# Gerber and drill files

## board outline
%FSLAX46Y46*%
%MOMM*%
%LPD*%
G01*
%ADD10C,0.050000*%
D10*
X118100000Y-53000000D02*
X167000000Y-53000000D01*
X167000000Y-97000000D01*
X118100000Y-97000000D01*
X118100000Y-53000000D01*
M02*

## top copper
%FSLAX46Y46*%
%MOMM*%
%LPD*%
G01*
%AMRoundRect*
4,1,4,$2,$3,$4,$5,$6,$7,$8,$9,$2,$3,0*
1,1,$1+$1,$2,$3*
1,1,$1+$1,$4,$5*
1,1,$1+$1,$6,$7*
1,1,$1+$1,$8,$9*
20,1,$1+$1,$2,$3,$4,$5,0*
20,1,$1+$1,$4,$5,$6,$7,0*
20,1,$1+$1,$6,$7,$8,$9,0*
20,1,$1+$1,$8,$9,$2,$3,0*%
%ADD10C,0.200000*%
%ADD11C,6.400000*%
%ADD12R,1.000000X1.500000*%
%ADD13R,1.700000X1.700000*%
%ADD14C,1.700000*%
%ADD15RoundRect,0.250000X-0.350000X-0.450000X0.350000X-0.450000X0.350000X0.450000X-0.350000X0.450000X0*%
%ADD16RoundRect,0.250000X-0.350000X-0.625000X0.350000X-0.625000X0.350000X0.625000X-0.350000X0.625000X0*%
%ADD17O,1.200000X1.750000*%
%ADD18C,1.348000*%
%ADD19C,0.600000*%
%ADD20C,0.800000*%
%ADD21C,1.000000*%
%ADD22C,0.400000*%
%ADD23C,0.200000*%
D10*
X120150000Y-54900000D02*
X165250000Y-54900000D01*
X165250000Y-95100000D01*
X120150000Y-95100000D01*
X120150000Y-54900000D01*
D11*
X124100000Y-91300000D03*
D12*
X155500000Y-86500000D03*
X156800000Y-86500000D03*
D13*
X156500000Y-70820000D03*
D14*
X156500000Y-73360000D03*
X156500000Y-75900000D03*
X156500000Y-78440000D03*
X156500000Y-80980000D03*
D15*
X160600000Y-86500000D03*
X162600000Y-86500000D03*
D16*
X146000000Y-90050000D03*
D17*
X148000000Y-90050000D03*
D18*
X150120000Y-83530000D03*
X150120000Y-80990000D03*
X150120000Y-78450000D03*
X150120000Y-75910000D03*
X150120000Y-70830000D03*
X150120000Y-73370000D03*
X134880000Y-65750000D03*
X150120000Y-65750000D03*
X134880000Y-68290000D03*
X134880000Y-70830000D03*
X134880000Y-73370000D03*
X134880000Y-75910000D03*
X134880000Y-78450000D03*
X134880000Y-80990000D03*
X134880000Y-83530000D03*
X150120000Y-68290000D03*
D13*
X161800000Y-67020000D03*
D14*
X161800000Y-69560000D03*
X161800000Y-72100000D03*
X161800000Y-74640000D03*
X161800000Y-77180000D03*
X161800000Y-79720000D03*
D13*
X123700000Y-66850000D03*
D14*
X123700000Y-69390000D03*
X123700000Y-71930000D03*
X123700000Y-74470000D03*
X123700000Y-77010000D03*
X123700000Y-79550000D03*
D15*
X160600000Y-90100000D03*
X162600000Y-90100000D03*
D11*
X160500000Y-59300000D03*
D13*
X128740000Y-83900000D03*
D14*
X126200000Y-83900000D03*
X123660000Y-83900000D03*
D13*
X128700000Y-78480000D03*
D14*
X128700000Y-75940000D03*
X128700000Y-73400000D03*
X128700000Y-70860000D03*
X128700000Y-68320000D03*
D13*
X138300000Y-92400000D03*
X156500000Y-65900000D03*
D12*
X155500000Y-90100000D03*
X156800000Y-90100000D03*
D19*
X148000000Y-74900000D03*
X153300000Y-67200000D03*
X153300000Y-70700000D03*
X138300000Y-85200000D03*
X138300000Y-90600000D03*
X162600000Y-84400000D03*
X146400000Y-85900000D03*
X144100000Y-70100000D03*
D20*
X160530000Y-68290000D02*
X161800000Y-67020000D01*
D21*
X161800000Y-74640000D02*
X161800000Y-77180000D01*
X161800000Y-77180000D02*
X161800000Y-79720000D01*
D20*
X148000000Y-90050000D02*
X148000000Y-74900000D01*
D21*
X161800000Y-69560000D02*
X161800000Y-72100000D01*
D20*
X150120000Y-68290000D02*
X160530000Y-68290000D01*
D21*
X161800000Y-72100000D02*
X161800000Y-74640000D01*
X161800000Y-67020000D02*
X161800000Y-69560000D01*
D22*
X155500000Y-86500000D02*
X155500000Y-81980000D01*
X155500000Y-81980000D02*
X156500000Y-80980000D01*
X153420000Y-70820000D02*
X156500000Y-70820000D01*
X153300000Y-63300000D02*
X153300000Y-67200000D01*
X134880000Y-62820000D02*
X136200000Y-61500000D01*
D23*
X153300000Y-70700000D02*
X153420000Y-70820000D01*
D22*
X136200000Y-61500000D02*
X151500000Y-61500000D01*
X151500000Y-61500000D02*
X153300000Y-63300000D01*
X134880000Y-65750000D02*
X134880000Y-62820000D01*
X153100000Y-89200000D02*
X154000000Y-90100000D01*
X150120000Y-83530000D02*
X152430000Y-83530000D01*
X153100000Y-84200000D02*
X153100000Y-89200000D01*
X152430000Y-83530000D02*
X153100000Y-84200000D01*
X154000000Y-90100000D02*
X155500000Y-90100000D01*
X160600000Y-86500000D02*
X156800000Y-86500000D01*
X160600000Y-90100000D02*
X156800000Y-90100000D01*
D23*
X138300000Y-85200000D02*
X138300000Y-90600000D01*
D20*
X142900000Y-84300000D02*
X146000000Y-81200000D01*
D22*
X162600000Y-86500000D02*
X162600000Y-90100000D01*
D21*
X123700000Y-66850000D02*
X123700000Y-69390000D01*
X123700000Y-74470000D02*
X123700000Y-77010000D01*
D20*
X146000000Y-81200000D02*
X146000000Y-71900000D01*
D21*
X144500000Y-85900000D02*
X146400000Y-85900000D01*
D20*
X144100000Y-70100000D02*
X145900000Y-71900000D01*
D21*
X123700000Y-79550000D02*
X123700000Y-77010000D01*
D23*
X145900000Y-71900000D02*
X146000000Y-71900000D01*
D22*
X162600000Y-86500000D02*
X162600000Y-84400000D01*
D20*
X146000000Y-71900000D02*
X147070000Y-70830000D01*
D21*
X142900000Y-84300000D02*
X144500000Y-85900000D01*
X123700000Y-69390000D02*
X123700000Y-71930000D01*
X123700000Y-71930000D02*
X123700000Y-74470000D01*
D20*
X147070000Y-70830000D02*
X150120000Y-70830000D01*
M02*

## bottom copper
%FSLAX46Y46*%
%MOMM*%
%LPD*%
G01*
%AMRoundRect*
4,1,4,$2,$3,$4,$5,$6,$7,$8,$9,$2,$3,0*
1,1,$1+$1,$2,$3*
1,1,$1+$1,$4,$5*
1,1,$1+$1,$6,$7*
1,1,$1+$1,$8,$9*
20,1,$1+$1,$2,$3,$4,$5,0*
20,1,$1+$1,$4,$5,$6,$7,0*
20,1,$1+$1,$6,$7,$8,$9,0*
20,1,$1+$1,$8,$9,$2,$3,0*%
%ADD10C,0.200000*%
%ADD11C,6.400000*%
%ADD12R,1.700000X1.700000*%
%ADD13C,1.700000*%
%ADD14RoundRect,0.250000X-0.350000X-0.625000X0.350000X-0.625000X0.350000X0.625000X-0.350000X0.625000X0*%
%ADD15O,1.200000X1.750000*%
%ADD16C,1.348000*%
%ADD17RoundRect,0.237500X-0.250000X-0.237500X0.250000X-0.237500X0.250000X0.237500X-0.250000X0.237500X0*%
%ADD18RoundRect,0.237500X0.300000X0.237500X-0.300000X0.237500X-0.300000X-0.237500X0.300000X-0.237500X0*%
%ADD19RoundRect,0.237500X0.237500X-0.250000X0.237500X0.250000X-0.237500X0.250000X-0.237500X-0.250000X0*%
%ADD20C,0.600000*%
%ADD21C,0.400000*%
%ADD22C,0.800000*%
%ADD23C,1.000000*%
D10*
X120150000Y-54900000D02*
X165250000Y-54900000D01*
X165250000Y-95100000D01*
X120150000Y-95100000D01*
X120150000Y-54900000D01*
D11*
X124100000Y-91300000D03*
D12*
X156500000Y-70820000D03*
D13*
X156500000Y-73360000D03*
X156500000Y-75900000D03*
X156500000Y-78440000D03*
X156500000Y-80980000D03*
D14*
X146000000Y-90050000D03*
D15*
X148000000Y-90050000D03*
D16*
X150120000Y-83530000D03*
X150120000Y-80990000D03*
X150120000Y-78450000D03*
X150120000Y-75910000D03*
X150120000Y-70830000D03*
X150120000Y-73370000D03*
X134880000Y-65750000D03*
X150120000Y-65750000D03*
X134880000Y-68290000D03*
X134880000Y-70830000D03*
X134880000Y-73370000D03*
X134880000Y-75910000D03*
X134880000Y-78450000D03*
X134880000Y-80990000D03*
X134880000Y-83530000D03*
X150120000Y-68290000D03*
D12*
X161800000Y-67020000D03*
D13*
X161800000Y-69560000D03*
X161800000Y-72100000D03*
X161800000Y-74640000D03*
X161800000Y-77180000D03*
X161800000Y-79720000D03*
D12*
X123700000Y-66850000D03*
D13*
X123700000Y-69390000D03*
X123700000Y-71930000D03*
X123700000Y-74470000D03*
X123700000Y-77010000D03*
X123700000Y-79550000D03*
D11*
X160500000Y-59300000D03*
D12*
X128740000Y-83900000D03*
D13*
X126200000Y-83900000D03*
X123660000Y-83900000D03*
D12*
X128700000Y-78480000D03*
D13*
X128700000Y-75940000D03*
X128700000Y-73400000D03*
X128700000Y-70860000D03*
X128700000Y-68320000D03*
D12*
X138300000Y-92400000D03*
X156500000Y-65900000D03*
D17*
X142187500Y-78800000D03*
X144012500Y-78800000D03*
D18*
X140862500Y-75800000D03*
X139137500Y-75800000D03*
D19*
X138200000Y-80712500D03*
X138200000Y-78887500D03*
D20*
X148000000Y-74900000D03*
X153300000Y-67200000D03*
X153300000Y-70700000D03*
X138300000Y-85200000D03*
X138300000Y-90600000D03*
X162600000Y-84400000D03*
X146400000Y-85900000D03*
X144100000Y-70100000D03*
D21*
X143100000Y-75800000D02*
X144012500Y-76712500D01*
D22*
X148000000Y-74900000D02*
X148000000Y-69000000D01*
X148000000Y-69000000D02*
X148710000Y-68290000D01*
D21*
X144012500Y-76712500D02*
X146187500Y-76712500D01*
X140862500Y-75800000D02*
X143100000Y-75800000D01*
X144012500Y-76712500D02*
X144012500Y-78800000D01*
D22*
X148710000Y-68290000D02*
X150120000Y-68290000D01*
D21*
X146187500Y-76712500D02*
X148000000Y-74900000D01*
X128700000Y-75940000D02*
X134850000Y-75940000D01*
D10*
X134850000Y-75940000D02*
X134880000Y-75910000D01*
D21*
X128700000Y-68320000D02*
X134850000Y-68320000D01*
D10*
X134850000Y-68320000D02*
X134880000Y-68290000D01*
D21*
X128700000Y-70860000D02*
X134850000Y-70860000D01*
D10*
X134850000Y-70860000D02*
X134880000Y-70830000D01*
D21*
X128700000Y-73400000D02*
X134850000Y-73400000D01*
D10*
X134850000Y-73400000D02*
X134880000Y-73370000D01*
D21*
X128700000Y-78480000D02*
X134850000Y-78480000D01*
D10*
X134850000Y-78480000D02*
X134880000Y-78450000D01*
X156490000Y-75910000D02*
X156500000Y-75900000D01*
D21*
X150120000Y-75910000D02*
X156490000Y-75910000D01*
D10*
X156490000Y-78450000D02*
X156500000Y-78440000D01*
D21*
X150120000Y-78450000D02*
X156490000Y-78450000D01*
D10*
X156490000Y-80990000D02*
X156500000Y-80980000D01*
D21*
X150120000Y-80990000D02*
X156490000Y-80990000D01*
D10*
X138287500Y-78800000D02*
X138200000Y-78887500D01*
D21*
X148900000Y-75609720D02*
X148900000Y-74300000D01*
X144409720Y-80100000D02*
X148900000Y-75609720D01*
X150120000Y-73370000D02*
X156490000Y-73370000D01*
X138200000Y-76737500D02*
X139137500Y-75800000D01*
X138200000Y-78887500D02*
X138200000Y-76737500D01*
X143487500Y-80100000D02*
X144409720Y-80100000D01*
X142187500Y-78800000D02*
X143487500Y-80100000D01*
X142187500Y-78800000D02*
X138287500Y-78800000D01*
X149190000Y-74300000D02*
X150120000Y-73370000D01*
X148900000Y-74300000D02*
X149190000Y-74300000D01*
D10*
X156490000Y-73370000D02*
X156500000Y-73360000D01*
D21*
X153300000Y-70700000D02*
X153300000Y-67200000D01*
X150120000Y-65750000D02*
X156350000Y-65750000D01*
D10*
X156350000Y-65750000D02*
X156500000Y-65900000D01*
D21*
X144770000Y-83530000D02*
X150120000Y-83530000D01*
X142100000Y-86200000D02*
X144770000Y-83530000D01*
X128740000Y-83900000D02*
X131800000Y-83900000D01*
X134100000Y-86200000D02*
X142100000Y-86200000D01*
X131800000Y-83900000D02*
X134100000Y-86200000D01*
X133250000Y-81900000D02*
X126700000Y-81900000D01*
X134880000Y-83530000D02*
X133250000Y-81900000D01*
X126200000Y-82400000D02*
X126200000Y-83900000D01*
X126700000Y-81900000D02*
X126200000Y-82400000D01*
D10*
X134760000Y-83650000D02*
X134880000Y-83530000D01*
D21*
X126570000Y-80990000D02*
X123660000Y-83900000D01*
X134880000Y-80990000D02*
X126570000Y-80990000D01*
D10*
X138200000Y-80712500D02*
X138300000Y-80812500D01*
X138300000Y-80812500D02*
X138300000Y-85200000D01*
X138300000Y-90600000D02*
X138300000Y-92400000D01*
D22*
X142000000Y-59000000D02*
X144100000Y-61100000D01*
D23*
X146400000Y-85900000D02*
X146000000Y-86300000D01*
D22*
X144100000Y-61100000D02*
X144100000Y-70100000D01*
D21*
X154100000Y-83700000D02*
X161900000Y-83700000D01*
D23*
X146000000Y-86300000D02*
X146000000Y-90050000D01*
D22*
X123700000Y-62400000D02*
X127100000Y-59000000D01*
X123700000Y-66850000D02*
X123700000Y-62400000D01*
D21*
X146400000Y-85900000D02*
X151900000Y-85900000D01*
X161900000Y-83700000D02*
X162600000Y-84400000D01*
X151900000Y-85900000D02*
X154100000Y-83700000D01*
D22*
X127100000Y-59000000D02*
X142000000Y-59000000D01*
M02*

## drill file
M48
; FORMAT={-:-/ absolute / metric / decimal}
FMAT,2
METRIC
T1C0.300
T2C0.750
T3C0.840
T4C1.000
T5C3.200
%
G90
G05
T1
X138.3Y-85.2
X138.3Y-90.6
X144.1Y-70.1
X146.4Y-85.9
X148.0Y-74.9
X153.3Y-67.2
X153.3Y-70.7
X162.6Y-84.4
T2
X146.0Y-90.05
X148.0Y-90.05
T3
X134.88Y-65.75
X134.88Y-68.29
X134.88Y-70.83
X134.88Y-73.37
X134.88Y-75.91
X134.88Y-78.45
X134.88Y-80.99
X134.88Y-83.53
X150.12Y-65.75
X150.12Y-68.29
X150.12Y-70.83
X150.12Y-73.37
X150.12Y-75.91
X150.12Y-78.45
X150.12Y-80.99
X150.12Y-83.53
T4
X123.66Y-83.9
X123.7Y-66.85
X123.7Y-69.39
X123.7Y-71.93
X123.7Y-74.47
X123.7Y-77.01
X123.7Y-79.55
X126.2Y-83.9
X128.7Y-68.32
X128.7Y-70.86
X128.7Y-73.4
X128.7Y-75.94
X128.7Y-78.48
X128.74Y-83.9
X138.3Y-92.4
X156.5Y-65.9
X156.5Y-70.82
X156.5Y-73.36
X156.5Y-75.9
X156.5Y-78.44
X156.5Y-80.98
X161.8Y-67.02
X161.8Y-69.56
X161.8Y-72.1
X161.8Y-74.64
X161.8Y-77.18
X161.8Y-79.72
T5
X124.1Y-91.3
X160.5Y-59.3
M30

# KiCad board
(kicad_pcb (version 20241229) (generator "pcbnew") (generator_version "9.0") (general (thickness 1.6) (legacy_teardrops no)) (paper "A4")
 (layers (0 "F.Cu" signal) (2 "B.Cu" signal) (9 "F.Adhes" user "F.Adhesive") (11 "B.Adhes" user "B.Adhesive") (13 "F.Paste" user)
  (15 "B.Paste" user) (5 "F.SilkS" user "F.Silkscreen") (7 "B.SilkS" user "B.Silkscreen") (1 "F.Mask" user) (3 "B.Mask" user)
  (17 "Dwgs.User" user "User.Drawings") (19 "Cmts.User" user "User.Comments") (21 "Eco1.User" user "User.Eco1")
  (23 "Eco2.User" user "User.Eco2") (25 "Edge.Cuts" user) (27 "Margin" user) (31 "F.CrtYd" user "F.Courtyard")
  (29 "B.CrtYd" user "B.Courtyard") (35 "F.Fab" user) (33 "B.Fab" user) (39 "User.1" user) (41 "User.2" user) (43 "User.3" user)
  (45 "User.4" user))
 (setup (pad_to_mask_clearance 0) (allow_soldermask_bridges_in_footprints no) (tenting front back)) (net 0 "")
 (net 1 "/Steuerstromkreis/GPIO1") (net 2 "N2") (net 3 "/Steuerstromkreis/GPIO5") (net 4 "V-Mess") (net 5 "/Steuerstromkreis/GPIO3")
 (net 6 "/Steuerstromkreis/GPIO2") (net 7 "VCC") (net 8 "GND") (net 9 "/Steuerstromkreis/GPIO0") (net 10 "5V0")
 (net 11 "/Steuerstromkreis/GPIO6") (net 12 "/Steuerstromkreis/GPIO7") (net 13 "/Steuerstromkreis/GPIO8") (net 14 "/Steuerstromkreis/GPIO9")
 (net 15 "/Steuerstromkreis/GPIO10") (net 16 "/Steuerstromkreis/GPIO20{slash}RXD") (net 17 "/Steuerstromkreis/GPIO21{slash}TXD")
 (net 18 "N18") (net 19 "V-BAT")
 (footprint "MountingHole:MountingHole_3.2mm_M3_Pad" (layer "F.Cu") (at 124.1 91.3)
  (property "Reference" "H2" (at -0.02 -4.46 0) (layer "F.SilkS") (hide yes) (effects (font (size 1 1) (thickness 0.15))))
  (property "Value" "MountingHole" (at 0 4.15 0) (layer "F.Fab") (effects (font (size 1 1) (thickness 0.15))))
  (pad "1" thru_hole circle (at 0 0) (size 6.4 6.4) (drill 3.2) (layers "*.Cu" "*.Mask") (remove_unused_layers no) (zone_connect 2)))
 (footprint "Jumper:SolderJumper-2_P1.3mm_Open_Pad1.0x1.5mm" (layer "F.Cu") (at 156.15 86.5)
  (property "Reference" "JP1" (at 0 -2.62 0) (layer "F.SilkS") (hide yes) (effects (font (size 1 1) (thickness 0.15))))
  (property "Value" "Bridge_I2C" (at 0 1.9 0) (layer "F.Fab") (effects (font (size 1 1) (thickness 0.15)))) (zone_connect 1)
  (pad "1" smd rect (at -0.65 0) (size 1 1.5) (layers "F.Cu" "F.Mask") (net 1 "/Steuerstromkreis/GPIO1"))
  (pad "2" smd rect (at 0.65 0) (size 1 1.5) (layers "F.Cu" "F.Mask") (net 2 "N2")))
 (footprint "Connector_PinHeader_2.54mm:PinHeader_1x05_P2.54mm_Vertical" (layer "F.Cu") (at 156.5 70.82)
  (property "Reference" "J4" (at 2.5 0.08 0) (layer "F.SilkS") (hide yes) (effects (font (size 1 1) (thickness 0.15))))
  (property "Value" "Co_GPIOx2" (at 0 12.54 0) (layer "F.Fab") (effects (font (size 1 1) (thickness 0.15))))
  (pad "1" thru_hole rect (at 0 0) (size 1.7 1.7) (drill 1) (layers "*.Cu" "*.Mask") (remove_unused_layers no)
   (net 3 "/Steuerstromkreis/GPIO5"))
  (pad "2" thru_hole circle (at 0 2.54) (size 1.7 1.7) (drill 1) (layers "*.Cu" "*.Mask") (remove_unused_layers no) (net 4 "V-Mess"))
  (pad "3" thru_hole circle (at 0 5.08) (size 1.7 1.7) (drill 1) (layers "*.Cu" "*.Mask") (remove_unused_layers no)
   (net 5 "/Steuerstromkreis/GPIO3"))
  (pad "4" thru_hole circle (at 0 7.62) (size 1.7 1.7) (drill 1) (layers "*.Cu" "*.Mask") (remove_unused_layers no)
   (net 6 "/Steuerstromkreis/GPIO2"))
  (pad "5" thru_hole circle (at 0 10.16) (size 1.7 1.7) (drill 1) (layers "*.Cu" "*.Mask") (remove_unused_layers no)
   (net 1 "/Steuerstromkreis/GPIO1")))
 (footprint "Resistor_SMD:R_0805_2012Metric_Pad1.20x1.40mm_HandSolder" (layer "F.Cu") (at 161.6 86.5)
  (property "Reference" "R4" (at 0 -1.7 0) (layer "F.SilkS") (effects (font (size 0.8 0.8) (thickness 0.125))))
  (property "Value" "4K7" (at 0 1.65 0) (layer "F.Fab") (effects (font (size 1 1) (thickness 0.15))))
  (pad "1" smd roundrect (at -1 0) (size 1.2 1.4) (layers "F.Cu" "F.Mask" "F.Paste") (roundrect_rratio 0.208333) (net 2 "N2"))
  (pad "2" smd roundrect (at 1 0) (size 1.2 1.4) (layers "F.Cu" "F.Mask" "F.Paste") (roundrect_rratio 0.208333) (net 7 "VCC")))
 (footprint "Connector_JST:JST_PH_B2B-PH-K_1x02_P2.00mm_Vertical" (layer "F.Cu") (at 146 90.05)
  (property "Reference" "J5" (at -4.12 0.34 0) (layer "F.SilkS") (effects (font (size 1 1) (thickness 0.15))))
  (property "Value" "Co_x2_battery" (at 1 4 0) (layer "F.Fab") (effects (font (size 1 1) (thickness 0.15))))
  (pad "1" thru_hole roundrect (at 0 0) (size 1.2 1.75) (drill 0.75) (layers "*.Cu" "*.Mask") (remove_unused_layers no)
   (roundrect_rratio 0.208333) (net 7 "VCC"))
  (pad "2" thru_hole oval (at 2 0) (size 1.2 1.75) (drill 0.75) (layers "*.Cu" "*.Mask") (remove_unused_layers no) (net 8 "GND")))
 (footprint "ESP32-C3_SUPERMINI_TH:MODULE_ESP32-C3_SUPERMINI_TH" (layer "F.Cu") (at 142.5 75.65)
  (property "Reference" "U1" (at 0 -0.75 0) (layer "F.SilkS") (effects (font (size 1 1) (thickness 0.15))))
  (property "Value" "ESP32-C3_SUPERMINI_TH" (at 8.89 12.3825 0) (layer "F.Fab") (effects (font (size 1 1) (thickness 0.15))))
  (pad "0" thru_hole circle (at 7.62 7.88) (size 1.348 1.348) (drill 0.84) (layers "*.Cu" "*.Mask") (remove_unused_layers no)
   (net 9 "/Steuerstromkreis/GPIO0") (solder_mask_margin 0.102))
  (pad "1" thru_hole circle (at 7.62 5.34) (size 1.348 1.348) (drill 0.84) (layers "*.Cu" "*.Mask") (remove_unused_layers no)
   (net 1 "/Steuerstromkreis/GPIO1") (solder_mask_margin 0.102))
  (pad "2" thru_hole circle (at 7.62 2.8) (size 1.348 1.348) (drill 0.84) (layers "*.Cu" "*.Mask") (remove_unused_layers no)
   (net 6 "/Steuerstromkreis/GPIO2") (solder_mask_margin 0.102))
  (pad "3" thru_hole circle (at 7.62 0.26) (size 1.348 1.348) (drill 0.84) (layers "*.Cu" "*.Mask") (remove_unused_layers no)
   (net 5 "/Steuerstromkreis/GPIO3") (solder_mask_margin 0.102))
  (pad "3.3" thru_hole circle (at 7.62 -4.82) (size 1.348 1.348) (drill 0.84) (layers "*.Cu" "*.Mask") (remove_unused_layers no)
   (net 7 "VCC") (solder_mask_margin 0.102))
  (pad "4" thru_hole circle (at 7.62 -2.28) (size 1.348 1.348) (drill 0.84) (layers "*.Cu" "*.Mask") (remove_unused_layers no)
   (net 4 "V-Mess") (solder_mask_margin 0.102))
  (pad "5" thru_hole circle (at -7.62 -9.9) (size 1.348 1.348) (drill 0.84) (layers "*.Cu" "*.Mask") (remove_unused_layers no)
   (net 3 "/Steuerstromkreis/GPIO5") (solder_mask_margin 0.102))
  (pad "5V" thru_hole circle (at 7.62 -9.9) (size 1.348 1.348) (drill 0.84) (layers "*.Cu" "*.Mask") (remove_unused_layers no)
   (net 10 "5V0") (solder_mask_margin 0.102))
  (pad "6" thru_hole circle (at -7.62 -7.36) (size 1.348 1.348) (drill 0.84) (layers "*.Cu" "*.Mask") (remove_unused_layers no)
   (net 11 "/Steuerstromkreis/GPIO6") (solder_mask_margin 0.102))
  (pad "7" thru_hole circle (at -7.62 -4.82) (size 1.348 1.348) (drill 0.84) (layers "*.Cu" "*.Mask") (remove_unused_layers no)
   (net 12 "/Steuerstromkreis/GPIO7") (solder_mask_margin 0.102))
  (pad "8" thru_hole circle (at -7.62 -2.28) (size 1.348 1.348) (drill 0.84) (layers "*.Cu" "*.Mask") (remove_unused_layers no)
   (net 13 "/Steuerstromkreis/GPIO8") (solder_mask_margin 0.102))
  (pad "9" thru_hole circle (at -7.62 0.26) (size 1.348 1.348) (drill 0.84) (layers "*.Cu" "*.Mask") (remove_unused_layers no)
   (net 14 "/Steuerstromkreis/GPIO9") (solder_mask_margin 0.102))
  (pad "10" thru_hole circle (at -7.62 2.8) (size 1.348 1.348) (drill 0.84) (layers "*.Cu" "*.Mask") (remove_unused_layers no)
   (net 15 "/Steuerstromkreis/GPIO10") (solder_mask_margin 0.102))
  (pad "20" thru_hole circle (at -7.62 5.34) (size 1.348 1.348) (drill 0.84) (layers "*.Cu" "*.Mask") (remove_unused_layers no)
   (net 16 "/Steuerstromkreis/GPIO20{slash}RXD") (solder_mask_margin 0.102))
  (pad "21" thru_hole circle (at -7.62 7.88) (size 1.348 1.348) (drill 0.84) (layers "*.Cu" "*.Mask") (remove_unused_layers no)
   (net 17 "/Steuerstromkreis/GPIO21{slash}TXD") (solder_mask_margin 0.102))
  (pad "G" thru_hole circle (at 7.62 -7.36) (size 1.348 1.348) (drill 0.84) (layers "*.Cu" "*.Mask") (remove_unused_layers no) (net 8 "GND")
   (solder_mask_margin 0.102)))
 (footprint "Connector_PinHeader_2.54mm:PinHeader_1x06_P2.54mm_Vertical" (layer "F.Cu") (at 161.8 67.02)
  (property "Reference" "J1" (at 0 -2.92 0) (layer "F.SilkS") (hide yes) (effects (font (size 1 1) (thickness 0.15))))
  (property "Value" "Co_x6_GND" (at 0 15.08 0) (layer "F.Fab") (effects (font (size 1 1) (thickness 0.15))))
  (pad "1" thru_hole rect (at 0 0) (size 1.7 1.7) (drill 1) (layers "*.Cu" "*.Mask") (remove_unused_layers no) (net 8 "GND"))
  (pad "2" thru_hole circle (at 0 2.54) (size 1.7 1.7) (drill 1) (layers "*.Cu" "*.Mask") (remove_unused_layers no) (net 8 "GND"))
  (pad "3" thru_hole circle (at 0 5.08) (size 1.7 1.7) (drill 1) (layers "*.Cu" "*.Mask") (remove_unused_layers no) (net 8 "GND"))
  (pad "4" thru_hole circle (at 0 7.62) (size 1.7 1.7) (drill 1) (layers "*.Cu" "*.Mask") (remove_unused_layers no) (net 8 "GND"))
  (pad "5" thru_hole circle (at 0 10.16) (size 1.7 1.7) (drill 1) (layers "*.Cu" "*.Mask") (remove_unused_layers no) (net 8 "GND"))
  (pad "6" thru_hole circle (at 0 12.7) (size 1.7 1.7) (drill 1) (layers "*.Cu" "*.Mask") (remove_unused_layers no) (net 8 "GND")))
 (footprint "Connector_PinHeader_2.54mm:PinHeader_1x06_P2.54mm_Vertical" (layer "F.Cu") (at 123.7 66.85)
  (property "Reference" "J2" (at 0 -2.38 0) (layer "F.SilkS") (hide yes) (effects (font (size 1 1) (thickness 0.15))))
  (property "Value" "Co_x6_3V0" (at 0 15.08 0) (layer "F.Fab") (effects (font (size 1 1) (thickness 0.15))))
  (pad "1" thru_hole rect (at 0 0) (size 1.7 1.7) (drill 1) (layers "*.Cu" "*.Mask") (remove_unused_layers no) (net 7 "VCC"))
  (pad "2" thru_hole circle (at 0 2.54) (size 1.7 1.7) (drill 1) (layers "*.Cu" "*.Mask") (remove_unused_layers no) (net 7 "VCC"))
  (pad "3" thru_hole circle (at 0 5.08) (size 1.7 1.7) (drill 1) (layers "*.Cu" "*.Mask") (remove_unused_layers no) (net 7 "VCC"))
  (pad "4" thru_hole circle (at 0 7.62) (size 1.7 1.7) (drill 1) (layers "*.Cu" "*.Mask") (remove_unused_layers no) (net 7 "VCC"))
  (pad "5" thru_hole circle (at 0 10.16) (size 1.7 1.7) (drill 1) (layers "*.Cu" "*.Mask") (remove_unused_layers no) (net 7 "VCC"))
  (pad "6" thru_hole circle (at 0 12.7) (size 1.7 1.7) (drill 1) (layers "*.Cu" "*.Mask") (remove_unused_layers no) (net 7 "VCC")))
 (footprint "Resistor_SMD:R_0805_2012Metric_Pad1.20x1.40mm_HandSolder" (layer "F.Cu") (at 161.6 90.1)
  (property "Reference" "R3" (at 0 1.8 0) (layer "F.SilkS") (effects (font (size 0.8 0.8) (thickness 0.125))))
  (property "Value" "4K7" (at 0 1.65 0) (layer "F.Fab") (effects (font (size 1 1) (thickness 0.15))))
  (pad "1" smd roundrect (at -1 0) (size 1.2 1.4) (layers "F.Cu" "F.Mask" "F.Paste") (roundrect_rratio 0.208333) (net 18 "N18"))
  (pad "2" smd roundrect (at 1 0) (size 1.2 1.4) (layers "F.Cu" "F.Mask" "F.Paste") (roundrect_rratio 0.208333) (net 7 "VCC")))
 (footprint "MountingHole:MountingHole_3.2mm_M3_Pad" (layer "F.Cu") (at 160.5 59.3)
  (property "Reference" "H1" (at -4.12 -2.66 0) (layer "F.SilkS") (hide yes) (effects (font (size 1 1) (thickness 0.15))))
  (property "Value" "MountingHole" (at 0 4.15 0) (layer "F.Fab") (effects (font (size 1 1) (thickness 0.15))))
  (pad "1" thru_hole circle (at 0 0) (size 6.4 6.4) (drill 3.2) (layers "*.Cu" "*.Mask") (remove_unused_layers no) (zone_connect 2)))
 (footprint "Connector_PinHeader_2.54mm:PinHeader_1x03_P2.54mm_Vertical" (layer "F.Cu") (at 128.74 83.9 -90)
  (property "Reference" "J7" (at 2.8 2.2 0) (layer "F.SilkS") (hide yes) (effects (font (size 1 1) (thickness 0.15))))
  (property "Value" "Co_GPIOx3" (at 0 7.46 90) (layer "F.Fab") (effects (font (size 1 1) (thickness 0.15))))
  (pad "1" thru_hole rect (at 0 0 270) (size 1.7 1.7) (drill 1) (layers "*.Cu" "*.Mask") (remove_unused_layers no)
   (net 9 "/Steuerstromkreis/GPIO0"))
  (pad "2" thru_hole circle (at 0 2.54 270) (size 1.7 1.7) (drill 1) (layers "*.Cu" "*.Mask") (remove_unused_layers no)
   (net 17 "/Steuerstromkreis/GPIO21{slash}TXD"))
  (pad "3" thru_hole circle (at 0 5.08 270) (size 1.7 1.7) (drill 1) (layers "*.Cu" "*.Mask") (remove_unused_layers no)
   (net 16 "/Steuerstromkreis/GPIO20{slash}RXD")))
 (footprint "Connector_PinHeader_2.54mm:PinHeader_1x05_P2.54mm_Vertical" (layer "F.Cu") (at 128.7 78.48 180)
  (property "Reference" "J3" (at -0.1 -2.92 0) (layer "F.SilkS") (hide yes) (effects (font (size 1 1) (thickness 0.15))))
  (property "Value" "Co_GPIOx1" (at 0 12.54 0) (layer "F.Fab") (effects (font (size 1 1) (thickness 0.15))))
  (pad "1" thru_hole rect (at 0 0 180) (size 1.7 1.7) (drill 1) (layers "*.Cu" "*.Mask") (remove_unused_layers no)
   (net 15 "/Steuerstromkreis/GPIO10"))
  (pad "2" thru_hole circle (at 0 2.54 180) (size 1.7 1.7) (drill 1) (layers "*.Cu" "*.Mask") (remove_unused_layers no)
   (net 14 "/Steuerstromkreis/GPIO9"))
  (pad "3" thru_hole circle (at 0 5.08 180) (size 1.7 1.7) (drill 1) (layers "*.Cu" "*.Mask") (remove_unused_layers no)
   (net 13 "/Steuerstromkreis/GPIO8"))
  (pad "4" thru_hole circle (at 0 7.62 180) (size 1.7 1.7) (drill 1) (layers "*.Cu" "*.Mask") (remove_unused_layers no)
   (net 12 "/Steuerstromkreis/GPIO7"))
  (pad "5" thru_hole circle (at 0 10.16 180) (size 1.7 1.7) (drill 1) (layers "*.Cu" "*.Mask") (remove_unused_layers no)
   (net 11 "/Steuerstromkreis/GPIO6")))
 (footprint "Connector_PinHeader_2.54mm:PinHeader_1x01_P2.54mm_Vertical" (layer "F.Cu") (at 138.3 92.4)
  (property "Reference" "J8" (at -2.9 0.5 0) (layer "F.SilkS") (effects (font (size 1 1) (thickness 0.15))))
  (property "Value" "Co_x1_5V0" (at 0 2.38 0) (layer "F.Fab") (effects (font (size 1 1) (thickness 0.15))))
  (pad "1" thru_hole rect (at 0 0) (size 1.7 1.7) (drill 1) (layers "*.Cu" "*.Mask") (remove_unused_layers no) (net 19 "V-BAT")))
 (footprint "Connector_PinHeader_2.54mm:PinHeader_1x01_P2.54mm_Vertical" (layer "F.Cu") (at 156.5 65.9)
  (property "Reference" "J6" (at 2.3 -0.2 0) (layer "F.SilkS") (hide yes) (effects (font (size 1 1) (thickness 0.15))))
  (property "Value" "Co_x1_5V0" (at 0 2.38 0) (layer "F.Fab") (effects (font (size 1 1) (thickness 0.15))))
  (pad "1" thru_hole rect (at 0 0) (size 1.7 1.7) (drill 1) (layers "*.Cu" "*.Mask") (remove_unused_layers no) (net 10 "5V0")))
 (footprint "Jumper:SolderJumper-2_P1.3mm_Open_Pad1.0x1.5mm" (layer "F.Cu") (at 156.15 90.1)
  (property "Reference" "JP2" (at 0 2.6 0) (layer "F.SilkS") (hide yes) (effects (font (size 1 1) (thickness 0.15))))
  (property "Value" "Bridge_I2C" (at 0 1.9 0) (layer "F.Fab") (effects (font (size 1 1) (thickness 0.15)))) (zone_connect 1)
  (pad "1" smd rect (at -0.65 0) (size 1 1.5) (layers "F.Cu" "F.Mask") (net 9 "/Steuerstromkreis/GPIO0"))
  (pad "2" smd rect (at 0.65 0) (size 1 1.5) (layers "F.Cu" "F.Mask") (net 18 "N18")))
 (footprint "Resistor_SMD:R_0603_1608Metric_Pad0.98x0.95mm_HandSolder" (layer "B.Cu") (at 143.1 78.8)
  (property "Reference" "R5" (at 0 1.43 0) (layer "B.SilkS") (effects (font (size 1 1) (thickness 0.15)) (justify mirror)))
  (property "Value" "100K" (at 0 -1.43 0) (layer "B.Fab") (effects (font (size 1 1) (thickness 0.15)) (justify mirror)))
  (pad "1" smd roundrect (at -0.9125 0) (size 0.975 0.95) (layers "B.Cu" "B.Mask" "B.Paste") (roundrect_rratio 0.25) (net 4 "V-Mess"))
  (pad "2" smd roundrect (at 0.9125 0) (size 0.975 0.95) (layers "B.Cu" "B.Mask" "B.Paste") (roundrect_rratio 0.25) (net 8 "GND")))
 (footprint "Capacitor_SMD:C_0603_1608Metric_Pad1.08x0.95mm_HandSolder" (layer "B.Cu") (at 140 75.8 180)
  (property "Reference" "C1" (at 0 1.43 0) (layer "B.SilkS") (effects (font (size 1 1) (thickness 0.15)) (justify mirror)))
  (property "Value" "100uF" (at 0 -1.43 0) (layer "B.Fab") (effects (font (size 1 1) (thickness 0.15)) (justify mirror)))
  (pad "1" smd roundrect (at -0.8625 0 180) (size 1.075 0.95) (layers "B.Cu" "B.Mask" "B.Paste") (roundrect_rratio 0.25) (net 8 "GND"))
  (pad "2" smd roundrect (at 0.8625 0 180) (size 1.075 0.95) (layers "B.Cu" "B.Mask" "B.Paste") (roundrect_rratio 0.25) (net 4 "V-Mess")))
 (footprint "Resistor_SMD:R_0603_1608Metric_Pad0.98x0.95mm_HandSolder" (layer "B.Cu") (at 138.2 79.8 90)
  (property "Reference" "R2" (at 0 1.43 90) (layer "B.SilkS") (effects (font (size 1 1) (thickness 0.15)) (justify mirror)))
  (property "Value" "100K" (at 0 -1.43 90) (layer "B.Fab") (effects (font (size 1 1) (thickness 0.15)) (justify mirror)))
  (pad "1" smd roundrect (at -0.9125 0 90) (size 0.975 0.95) (layers "B.Cu" "B.Mask" "B.Paste") (roundrect_rratio 0.25) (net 19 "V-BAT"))
  (pad "2" smd roundrect (at 0.9125 0 90) (size 0.975 0.95) (layers "B.Cu" "B.Mask" "B.Paste") (roundrect_rratio 0.25) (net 4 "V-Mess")))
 (gr_rect (start 120.15 54.9) (end 165.25 95.1) (stroke (width 0.2) (type default)) (fill no) (layer "F.Cu"))
 (gr_rect (start 120.15 54.9) (end 165.25 95.1) (stroke (width 0.2) (type default)) (fill no) (layer "B.Cu") (net 16))
 (gr_rect (start 118.1 53) (end 167 97) (stroke (width 0.05) (type default)) (fill no) (layer "Edge.Cuts"))
 (segment (start 160.53 68.29) (end 161.8 67.02) (width 0.8) (layer "F.Cu") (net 8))
 (segment (start 161.8 74.64) (end 161.8 77.18) (width 1) (layer "F.Cu") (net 8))
 (segment (start 161.8 77.18) (end 161.8 79.72) (width 1) (layer "F.Cu") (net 8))
 (segment (start 148 90.05) (end 148 74.9) (width 0.8) (layer "F.Cu") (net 8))
 (segment (start 161.8 69.56) (end 161.8 72.1) (width 1) (layer "F.Cu") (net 8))
 (segment (start 150.12 68.29) (end 160.53 68.29) (width 0.8) (layer "F.Cu") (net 8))
 (segment (start 161.8 72.1) (end 161.8 74.64) (width 1) (layer "F.Cu") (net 8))
 (segment (start 161.8 67.02) (end 161.8 69.56) (width 1) (layer "F.Cu") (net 8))
 (via (at 148 74.9) (size 0.6) (drill 0.3) (layers "F.Cu" "B.Cu") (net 8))
 (segment (start 143.1 75.8) (end 144.0125 76.7125) (width 0.4) (layer "B.Cu") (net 8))
 (segment (start 148 74.9) (end 148 69) (width 0.8) (layer "B.Cu") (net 8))
 (segment (start 148 69) (end 148.71 68.29) (width 0.8) (layer "B.Cu") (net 8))
 (segment (start 144.0125 76.7125) (end 146.1875 76.7125) (width 0.4) (layer "B.Cu") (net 8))
 (segment (start 140.8625 75.8) (end 143.1 75.8) (width 0.4) (layer "B.Cu") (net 8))
 (segment (start 144.0125 76.7125) (end 144.0125 78.8) (width 0.4) (layer "B.Cu") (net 8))
 (segment (start 148.71 68.29) (end 150.12 68.29) (width 0.8) (layer "B.Cu") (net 8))
 (segment (start 146.1875 76.7125) (end 148 74.9) (width 0.4) (layer "B.Cu") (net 8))
 (segment (start 128.7 75.94) (end 134.85 75.94) (width 0.4) (layer "B.Cu") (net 14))
 (segment (start 134.85 75.94) (end 134.88 75.91) (width 0.2) (layer "B.Cu") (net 14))
 (segment (start 128.7 68.32) (end 134.85 68.32) (width 0.4) (layer "B.Cu") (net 11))
 (segment (start 134.85 68.32) (end 134.88 68.29) (width 0.2) (layer "B.Cu") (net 11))
 (segment (start 128.7 70.86) (end 134.85 70.86) (width 0.4) (layer "B.Cu") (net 12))
 (segment (start 134.85 70.86) (end 134.88 70.83) (width 0.2) (layer "B.Cu") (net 12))
 (segment (start 128.7 73.4) (end 134.85 73.4) (width 0.4) (layer "B.Cu") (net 13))
 (segment (start 134.85 73.4) (end 134.88 73.37) (width 0.2) (layer "B.Cu") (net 13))
 (segment (start 128.7 78.48) (end 134.85 78.48) (width 0.4) (layer "B.Cu") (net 15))
 (segment (start 134.85 78.48) (end 134.88 78.45) (width 0.2) (layer "B.Cu") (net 15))
 (segment (start 156.49 75.91) (end 156.5 75.9) (width 0.2) (layer "B.Cu") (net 5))
 (segment (start 150.12 75.91) (end 156.49 75.91) (width 0.4) (layer "B.Cu") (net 5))
 (segment (start 156.49 78.45) (end 156.5 78.44) (width 0.2) (layer "B.Cu") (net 6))
 (segment (start 150.12 78.45) (end 156.49 78.45) (width 0.4) (layer "B.Cu") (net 6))
 (segment (start 155.5 86.5) (end 155.5 81.98) (width 0.4) (layer "F.Cu") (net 1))
 (segment (start 155.5 81.98) (end 156.5 80.98) (width 0.4) (layer "F.Cu") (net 1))
 (segment (start 156.49 80.99) (end 156.5 80.98) (width 0.2) (layer "B.Cu") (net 1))
 (segment (start 150.12 80.99) (end 156.49 80.99) (width 0.4) (layer "B.Cu") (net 1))
 (segment (start 138.2875 78.8) (end 138.2 78.8875) (width 0.2) (layer "B.Cu") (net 4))
 (segment (start 148.9 75.60972) (end 148.9 74.3) (width 0.4) (layer "B.Cu") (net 4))
 (segment (start 144.40972 80.1) (end 148.9 75.60972) (width 0.4) (layer "B.Cu") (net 4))
 (segment (start 150.12 73.37) (end 156.49 73.37) (width 0.4) (layer "B.Cu") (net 4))
 (segment (start 138.2 76.7375) (end 139.1375 75.8) (width 0.4) (layer "B.Cu") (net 4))
 (segment (start 138.2 78.8875) (end 138.2 76.7375) (width 0.4) (layer "B.Cu") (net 4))
 (segment (start 143.4875 80.1) (end 144.40972 80.1) (width 0.4) (layer "B.Cu") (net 4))
 (segment (start 142.1875 78.8) (end 143.4875 80.1) (width 0.4) (layer "B.Cu") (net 4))
 (segment (start 142.1875 78.8) (end 138.2875 78.8) (width 0.4) (layer "B.Cu") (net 4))
 (segment (start 149.19 74.3) (end 150.12 73.37) (width 0.4) (layer "B.Cu") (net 4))
 (segment (start 148.9 74.3) (end 149.19 74.3) (width 0.4) (layer "B.Cu") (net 4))
 (segment (start 156.49 73.37) (end 156.5 73.36) (width 0.2) (layer "B.Cu") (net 4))
 (segment (start 153.42 70.82) (end 156.5 70.82) (width 0.4) (layer "F.Cu") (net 3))
 (segment (start 153.3 63.3) (end 153.3 67.2) (width 0.4) (layer "F.Cu") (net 3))
 (segment (start 134.88 62.82) (end 136.2 61.5) (width 0.4) (layer "F.Cu") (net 3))
 (segment (start 153.3 70.7) (end 153.42 70.82) (width 0.2) (layer "F.Cu") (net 3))
 (segment (start 136.2 61.5) (end 151.5 61.5) (width 0.4) (layer "F.Cu") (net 3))
 (segment (start 151.5 61.5) (end 153.3 63.3) (width 0.4) (layer "F.Cu") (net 3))
 (segment (start 134.88 65.75) (end 134.88 62.82) (width 0.4) (layer "F.Cu") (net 3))
 (via (at 153.3 67.2) (size 0.6) (drill 0.3) (layers "F.Cu" "B.Cu") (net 3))
 (via (at 153.3 70.7) (size 0.6) (drill 0.3) (layers "F.Cu" "B.Cu") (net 3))
 (segment (start 153.3 70.7) (end 153.3 67.2) (width 0.4) (layer "B.Cu") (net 3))
 (segment (start 150.12 65.75) (end 156.35 65.75) (width 0.4) (layer "B.Cu") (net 10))
 (segment (start 156.35 65.75) (end 156.5 65.9) (width 0.2) (layer "B.Cu") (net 10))
 (segment (start 153.1 89.2) (end 154 90.1) (width 0.4) (layer "F.Cu") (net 9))
 (segment (start 150.12 83.53) (end 152.43 83.53) (width 0.4) (layer "F.Cu") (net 9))
 (segment (start 153.1 84.2) (end 153.1 89.2) (width 0.4) (layer "F.Cu") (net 9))
 (segment (start 152.43 83.53) (end 153.1 84.2) (width 0.4) (layer "F.Cu") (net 9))
 (segment (start 154 90.1) (end 155.5 90.1) (width 0.4) (layer "F.Cu") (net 9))
 (segment (start 144.77 83.53) (end 150.12 83.53) (width 0.4) (layer "B.Cu") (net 9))
 (segment (start 142.1 86.2) (end 144.77 83.53) (width 0.4) (layer "B.Cu") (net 9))
 (segment (start 128.74 83.9) (end 131.8 83.9) (width 0.4) (layer "B.Cu") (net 9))
 (segment (start 134.1 86.2) (end 142.1 86.2) (width 0.4) (layer "B.Cu") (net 9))
 (segment (start 131.8 83.9) (end 134.1 86.2) (width 0.4) (layer "B.Cu") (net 9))
 (segment (start 133.25 81.9) (end 126.7 81.9) (width 0.4) (layer "B.Cu") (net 17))
 (segment (start 134.88 83.53) (end 133.25 81.9) (width 0.4) (layer "B.Cu") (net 17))
 (segment (start 126.2 82.4) (end 126.2 83.9) (width 0.4) (layer "B.Cu") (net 17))
 (segment (start 126.7 81.9) (end 126.2 82.4) (width 0.4) (layer "B.Cu") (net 17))
 (segment (start 134.76 83.65) (end 134.88 83.53) (width 0.2) (layer "B.Cu") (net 17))
 (segment (start 126.57 80.99) (end 123.66 83.9) (width 0.4) (layer "B.Cu") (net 16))
 (segment (start 134.88 80.99) (end 126.57 80.99) (width 0.4) (layer "B.Cu") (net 16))
 (segment (start 160.6 86.5) (end 156.8 86.5) (width 0.4) (layer "F.Cu") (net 2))
 (segment (start 160.6 90.1) (end 156.8 90.1) (width 0.4) (layer "F.Cu") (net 18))
 (segment (start 138.3 85.2) (end 138.3 90.6) (width 0.2) (layer "F.Cu") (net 19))
 (via (at 138.3 85.2) (size 0.6) (drill 0.3) (layers "F.Cu" "B.Cu") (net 19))
 (via (at 138.3 90.6) (size 0.6) (drill 0.3) (layers "F.Cu" "B.Cu") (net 19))
 (segment (start 138.2 80.7125) (end 138.3 80.8125) (width 0.2) (layer "B.Cu") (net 19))
 (segment (start 138.3 80.8125) (end 138.3 85.2) (width 0.2) (layer "B.Cu") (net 19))
 (segment (start 138.3 90.6) (end 138.3 92.4) (width 0.2) (layer "B.Cu") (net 19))
 (segment (start 142.9 84.3) (end 146 81.2) (width 0.8) (layer "F.Cu") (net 7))
 (segment (start 162.6 86.5) (end 162.6 90.1) (width 0.4) (layer "F.Cu") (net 7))
 (segment (start 123.7 66.85) (end 123.7 69.39) (width 1) (layer "F.Cu") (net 7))
 (segment (start 123.7 74.47) (end 123.7 77.01) (width 1) (layer "F.Cu") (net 7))
 (segment (start 146 81.2) (end 146 71.9) (width 0.8) (layer "F.Cu") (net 7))
 (segment (start 144.5 85.9) (end 146.4 85.9) (width 1) (layer "F.Cu") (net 7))
 (segment (start 144.1 70.1) (end 145.9 71.9) (width 0.8) (layer "F.Cu") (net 7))
 (segment (start 123.7 79.55) (end 123.7 77.01) (width 1) (layer "F.Cu") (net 7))
 (segment (start 145.9 71.9) (end 146 71.9) (width 0.2) (layer "F.Cu") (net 7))
 (segment (start 162.6 86.5) (end 162.6 84.4) (width 0.4) (layer "F.Cu") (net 7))
 (segment (start 146 71.9) (end 147.07 70.83) (width 0.8) (layer "F.Cu") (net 7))
 (segment (start 142.9 84.3) (end 144.5 85.9) (width 1) (layer "F.Cu") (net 7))
 (segment (start 123.7 69.39) (end 123.7 71.93) (width 1) (layer "F.Cu") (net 7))
 (segment (start 123.7 71.93) (end 123.7 74.47) (width 1) (layer "F.Cu") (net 7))
 (segment (start 147.07 70.83) (end 150.12 70.83) (width 0.8) (layer "F.Cu") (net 7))
 (via (at 162.6 84.4) (size 0.6) (drill 0.3) (layers "F.Cu" "B.Cu") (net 7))
 (via (at 146.4 85.9) (size 0.6) (drill 0.3) (layers "F.Cu" "B.Cu") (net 7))
 (via (at 144.1 70.1) (size 0.6) (drill 0.3) (layers "F.Cu" "B.Cu") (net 7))
 (segment (start 142 59) (end 144.1 61.1) (width 0.8) (layer "B.Cu") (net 7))
 (segment (start 146.4 85.9) (end 146 86.3) (width 1) (layer "B.Cu") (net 7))
 (segment (start 144.1 61.1) (end 144.1 70.1) (width 0.8) (layer "B.Cu") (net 7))
 (segment (start 154.1 83.7) (end 161.9 83.7) (width 0.4) (layer "B.Cu") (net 7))
 (segment (start 146 86.3) (end 146 90.05) (width 1) (layer "B.Cu") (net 7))
 (segment (start 123.7 62.4) (end 127.1 59) (width 0.8) (layer "B.Cu") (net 7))
 (segment (start 123.7 66.85) (end 123.7 62.4) (width 0.8) (layer "B.Cu") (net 7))
 (segment (start 146.4 85.9) (end 151.9 85.9) (width 0.4) (layer "B.Cu") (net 7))
 (segment (start 161.9 83.7) (end 162.6 84.4) (width 0.4) (layer "B.Cu") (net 7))
 (segment (start 151.9 85.9) (end 154.1 83.7) (width 0.4) (layer "B.Cu") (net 7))
 (segment (start 127.1 59) (end 142 59) (width 0.8) (layer "B.Cu") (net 7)))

